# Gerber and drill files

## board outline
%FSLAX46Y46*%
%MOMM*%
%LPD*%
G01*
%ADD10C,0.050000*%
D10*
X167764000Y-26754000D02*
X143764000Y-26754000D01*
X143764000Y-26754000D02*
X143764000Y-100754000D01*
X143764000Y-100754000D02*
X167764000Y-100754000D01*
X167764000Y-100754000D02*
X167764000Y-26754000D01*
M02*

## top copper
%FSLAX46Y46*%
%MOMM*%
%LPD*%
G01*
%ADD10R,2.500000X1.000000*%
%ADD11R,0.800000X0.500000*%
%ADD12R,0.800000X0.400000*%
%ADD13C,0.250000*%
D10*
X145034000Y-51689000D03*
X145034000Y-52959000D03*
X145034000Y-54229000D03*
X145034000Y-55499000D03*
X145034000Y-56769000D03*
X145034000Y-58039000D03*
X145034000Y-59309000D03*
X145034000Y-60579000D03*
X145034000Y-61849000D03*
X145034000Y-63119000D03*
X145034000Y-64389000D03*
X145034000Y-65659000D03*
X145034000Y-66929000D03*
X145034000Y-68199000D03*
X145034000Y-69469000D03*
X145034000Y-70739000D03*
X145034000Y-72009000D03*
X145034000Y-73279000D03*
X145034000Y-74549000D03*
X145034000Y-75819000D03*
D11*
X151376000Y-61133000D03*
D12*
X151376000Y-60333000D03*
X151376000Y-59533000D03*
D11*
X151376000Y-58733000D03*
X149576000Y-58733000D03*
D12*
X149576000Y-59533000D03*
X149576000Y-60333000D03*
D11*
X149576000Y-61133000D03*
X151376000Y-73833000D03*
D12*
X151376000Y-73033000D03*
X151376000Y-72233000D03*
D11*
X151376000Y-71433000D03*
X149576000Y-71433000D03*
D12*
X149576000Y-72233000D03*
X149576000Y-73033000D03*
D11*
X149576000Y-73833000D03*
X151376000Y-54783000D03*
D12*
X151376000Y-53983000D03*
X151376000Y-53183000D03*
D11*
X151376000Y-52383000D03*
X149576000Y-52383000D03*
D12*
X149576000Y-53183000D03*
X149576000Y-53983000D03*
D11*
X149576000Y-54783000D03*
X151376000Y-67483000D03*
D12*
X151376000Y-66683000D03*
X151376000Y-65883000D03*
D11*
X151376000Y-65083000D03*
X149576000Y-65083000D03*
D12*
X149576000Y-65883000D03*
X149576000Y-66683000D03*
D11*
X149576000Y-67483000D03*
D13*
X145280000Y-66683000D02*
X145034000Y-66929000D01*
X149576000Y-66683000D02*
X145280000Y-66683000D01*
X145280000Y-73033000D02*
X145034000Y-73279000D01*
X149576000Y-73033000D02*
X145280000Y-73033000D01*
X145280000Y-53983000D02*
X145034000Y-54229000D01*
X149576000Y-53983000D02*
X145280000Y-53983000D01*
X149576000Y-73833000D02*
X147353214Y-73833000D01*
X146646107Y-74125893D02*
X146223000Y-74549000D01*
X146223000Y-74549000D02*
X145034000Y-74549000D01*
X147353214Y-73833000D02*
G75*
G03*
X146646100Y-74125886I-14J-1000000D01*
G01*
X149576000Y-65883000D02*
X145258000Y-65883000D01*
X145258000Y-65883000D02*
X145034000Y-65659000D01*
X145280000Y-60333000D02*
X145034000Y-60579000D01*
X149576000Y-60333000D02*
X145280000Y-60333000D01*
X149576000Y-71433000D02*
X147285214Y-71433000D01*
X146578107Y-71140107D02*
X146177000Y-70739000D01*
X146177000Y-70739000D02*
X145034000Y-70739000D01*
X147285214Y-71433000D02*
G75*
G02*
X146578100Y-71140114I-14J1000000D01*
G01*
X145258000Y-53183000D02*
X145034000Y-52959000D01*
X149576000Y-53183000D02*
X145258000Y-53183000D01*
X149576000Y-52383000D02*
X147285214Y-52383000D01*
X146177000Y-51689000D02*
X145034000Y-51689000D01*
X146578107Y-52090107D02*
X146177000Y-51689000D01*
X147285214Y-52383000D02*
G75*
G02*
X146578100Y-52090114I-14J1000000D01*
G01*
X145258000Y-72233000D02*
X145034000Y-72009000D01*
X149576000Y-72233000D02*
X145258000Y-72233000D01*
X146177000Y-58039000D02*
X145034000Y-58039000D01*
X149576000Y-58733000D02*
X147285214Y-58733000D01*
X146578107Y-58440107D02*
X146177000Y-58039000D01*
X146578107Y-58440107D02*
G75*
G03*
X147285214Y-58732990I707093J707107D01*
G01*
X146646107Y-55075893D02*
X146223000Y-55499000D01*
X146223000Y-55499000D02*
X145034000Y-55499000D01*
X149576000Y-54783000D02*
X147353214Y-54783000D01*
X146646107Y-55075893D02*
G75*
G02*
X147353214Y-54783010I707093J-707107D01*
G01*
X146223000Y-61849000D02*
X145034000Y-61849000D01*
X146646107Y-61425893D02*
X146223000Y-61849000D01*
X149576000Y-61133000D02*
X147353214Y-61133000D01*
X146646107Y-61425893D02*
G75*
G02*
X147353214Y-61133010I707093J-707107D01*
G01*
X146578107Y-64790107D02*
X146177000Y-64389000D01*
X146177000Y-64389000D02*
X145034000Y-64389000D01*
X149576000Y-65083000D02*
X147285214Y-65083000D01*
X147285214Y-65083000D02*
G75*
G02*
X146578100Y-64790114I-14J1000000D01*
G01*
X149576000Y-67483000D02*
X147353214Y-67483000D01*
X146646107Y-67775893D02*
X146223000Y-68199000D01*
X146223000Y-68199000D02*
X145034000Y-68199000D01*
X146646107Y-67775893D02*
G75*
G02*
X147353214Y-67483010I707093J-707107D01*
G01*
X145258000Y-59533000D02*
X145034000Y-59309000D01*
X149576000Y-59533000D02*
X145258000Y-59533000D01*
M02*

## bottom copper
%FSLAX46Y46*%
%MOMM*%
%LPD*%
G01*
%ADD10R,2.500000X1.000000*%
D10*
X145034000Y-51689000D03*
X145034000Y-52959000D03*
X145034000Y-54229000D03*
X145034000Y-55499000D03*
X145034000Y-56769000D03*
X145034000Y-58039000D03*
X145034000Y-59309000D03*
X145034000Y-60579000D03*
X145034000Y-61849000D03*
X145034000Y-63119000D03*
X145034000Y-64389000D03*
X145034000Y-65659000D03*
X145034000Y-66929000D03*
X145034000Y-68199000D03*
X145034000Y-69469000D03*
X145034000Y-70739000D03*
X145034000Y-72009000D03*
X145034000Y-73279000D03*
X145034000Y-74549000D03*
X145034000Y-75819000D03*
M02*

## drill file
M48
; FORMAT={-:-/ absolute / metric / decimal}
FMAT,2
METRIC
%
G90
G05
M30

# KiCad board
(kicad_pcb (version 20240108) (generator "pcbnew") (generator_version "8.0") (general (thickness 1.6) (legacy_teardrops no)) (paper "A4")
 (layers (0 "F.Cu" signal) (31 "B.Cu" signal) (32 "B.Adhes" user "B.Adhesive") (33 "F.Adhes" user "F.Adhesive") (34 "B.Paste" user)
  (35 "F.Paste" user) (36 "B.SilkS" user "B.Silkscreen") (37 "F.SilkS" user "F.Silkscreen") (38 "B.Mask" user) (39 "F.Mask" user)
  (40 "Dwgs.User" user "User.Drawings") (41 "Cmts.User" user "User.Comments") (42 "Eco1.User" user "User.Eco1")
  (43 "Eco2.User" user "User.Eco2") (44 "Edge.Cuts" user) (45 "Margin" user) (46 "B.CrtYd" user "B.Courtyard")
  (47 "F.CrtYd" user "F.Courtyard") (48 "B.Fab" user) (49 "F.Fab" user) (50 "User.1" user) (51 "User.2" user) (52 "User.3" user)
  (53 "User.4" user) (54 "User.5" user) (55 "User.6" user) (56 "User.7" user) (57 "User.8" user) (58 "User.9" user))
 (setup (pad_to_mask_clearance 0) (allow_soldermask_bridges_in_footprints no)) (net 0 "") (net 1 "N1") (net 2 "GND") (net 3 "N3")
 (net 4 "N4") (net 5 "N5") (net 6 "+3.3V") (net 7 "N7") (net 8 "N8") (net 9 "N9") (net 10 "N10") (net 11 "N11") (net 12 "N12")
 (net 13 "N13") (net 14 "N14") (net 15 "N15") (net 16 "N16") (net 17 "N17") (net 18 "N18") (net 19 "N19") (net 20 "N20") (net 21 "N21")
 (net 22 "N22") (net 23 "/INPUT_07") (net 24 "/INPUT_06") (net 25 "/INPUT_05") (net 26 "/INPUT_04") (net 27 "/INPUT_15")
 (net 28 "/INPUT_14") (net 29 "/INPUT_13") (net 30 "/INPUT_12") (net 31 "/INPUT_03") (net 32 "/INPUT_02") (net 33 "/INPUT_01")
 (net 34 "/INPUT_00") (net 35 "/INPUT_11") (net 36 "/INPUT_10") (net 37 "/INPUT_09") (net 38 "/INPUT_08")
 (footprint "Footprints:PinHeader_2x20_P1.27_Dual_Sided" (layer "F.Cu") (at 145.034 63.754)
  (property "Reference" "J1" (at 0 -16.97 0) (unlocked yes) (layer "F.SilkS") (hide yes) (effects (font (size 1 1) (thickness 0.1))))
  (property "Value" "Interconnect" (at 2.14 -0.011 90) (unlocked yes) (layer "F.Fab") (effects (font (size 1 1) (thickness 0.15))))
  (pad "1" smd rect (at 0 -12.065 180) (size 2.5 1) (layers "F.Cu" "F.Paste" "F.Mask") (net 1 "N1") (thermal_bridge_angle 45))
  (pad "2" smd rect (at 0 -12.065 180) (size 2.5 1) (layers "B.Cu" "B.Paste" "B.Mask") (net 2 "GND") (thermal_bridge_angle 45))
  (pad "3" smd rect (at 0 -10.795 180) (size 2.5 1) (layers "F.Cu" "F.Paste" "F.Mask") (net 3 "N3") (thermal_bridge_angle 45))
  (pad "4" smd rect (at 0 -10.795 180) (size 2.5 1) (layers "B.Cu" "B.Paste" "B.Mask") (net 2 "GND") (thermal_bridge_angle 45))
  (pad "5" smd rect (at 0 -9.525 180) (size 2.5 1) (layers "F.Cu" "F.Paste" "F.Mask") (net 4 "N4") (thermal_bridge_angle 45))
  (pad "6" smd rect (at 0 -9.525 180) (size 2.5 1) (layers "B.Cu" "B.Paste" "B.Mask") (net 2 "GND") (thermal_bridge_angle 45))
  (pad "7" smd rect (at 0 -8.255 180) (size 2.5 1) (layers "F.Cu" "F.Paste" "F.Mask") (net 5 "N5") (thermal_bridge_angle 45))
  (pad "8" smd rect (at 0 -8.255 180) (size 2.5 1) (layers "B.Cu" "B.Paste" "B.Mask") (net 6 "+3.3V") (thermal_bridge_angle 45))
  (pad "9" smd rect (at 0 -6.985 180) (size 2.5 1) (layers "F.Cu" "F.Paste" "F.Mask") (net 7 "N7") (thermal_bridge_angle 45))
  (pad "10" smd rect (at 0 -6.985 180) (size 2.5 1) (layers "B.Cu" "B.Paste" "B.Mask") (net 2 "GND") (thermal_bridge_angle 45))
  (pad "11" smd rect (at 0 -5.715 180) (size 2.5 1) (layers "F.Cu" "F.Paste" "F.Mask") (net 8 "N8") (thermal_bridge_angle 45))
  (pad "12" smd rect (at 0 -5.715 180) (size 2.5 1) (layers "B.Cu" "B.Paste" "B.Mask") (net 2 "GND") (thermal_bridge_angle 45))
  (pad "13" smd rect (at 0 -4.445 180) (size 2.5 1) (layers "F.Cu" "F.Paste" "F.Mask") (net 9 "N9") (thermal_bridge_angle 45))
  (pad "14" smd rect (at 0 -4.445 180) (size 2.5 1) (layers "B.Cu" "B.Paste" "B.Mask") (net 2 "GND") (thermal_bridge_angle 45))
  (pad "15" smd rect (at 0 -3.175 180) (size 2.5 1) (layers "F.Cu" "F.Paste" "F.Mask") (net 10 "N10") (thermal_bridge_angle 45))
  (pad "16" smd rect (at 0 -3.175 180) (size 2.5 1) (layers "B.Cu" "B.Paste" "B.Mask") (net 2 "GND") (thermal_bridge_angle 45))
  (pad "17" smd rect (at 0 -1.905 180) (size 2.5 1) (layers "F.Cu" "F.Paste" "F.Mask") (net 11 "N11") (thermal_bridge_angle 45))
  (pad "18" smd rect (at 0 -1.905 180) (size 2.5 1) (layers "B.Cu" "B.Paste" "B.Mask") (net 6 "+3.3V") (thermal_bridge_angle 45))
  (pad "19" smd rect (at 0 -0.635 180) (size 2.5 1) (layers "F.Cu" "F.Paste" "F.Mask") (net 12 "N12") (thermal_bridge_angle 45))
  (pad "20" smd rect (at 0 -0.635 180) (size 2.5 1) (layers "B.Cu" "B.Paste" "B.Mask") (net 2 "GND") (thermal_bridge_angle 45))
  (pad "21" smd rect (at 0 0.635 180) (size 2.5 1) (layers "F.Cu" "F.Paste" "F.Mask") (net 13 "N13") (thermal_bridge_angle 45))
  (pad "22" smd rect (at 0 0.635 180) (size 2.5 1) (layers "B.Cu" "B.Paste" "B.Mask") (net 2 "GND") (thermal_bridge_angle 45))
  (pad "23" smd rect (at 0 1.905 180) (size 2.5 1) (layers "F.Cu" "F.Paste" "F.Mask") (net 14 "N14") (thermal_bridge_angle 45))
  (pad "24" smd rect (at 0 1.905 180) (size 2.5 1) (layers "B.Cu" "B.Paste" "B.Mask") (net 2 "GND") (thermal_bridge_angle 45))
  (pad "25" smd rect (at 0 3.175 180) (size 2.5 1) (layers "F.Cu" "F.Paste" "F.Mask") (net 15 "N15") (thermal_bridge_angle 45))
  (pad "26" smd rect (at 0 3.175 180) (size 2.5 1) (layers "B.Cu" "B.Paste" "B.Mask") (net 2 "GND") (thermal_bridge_angle 45))
  (pad "27" smd rect (at 0 4.445 180) (size 2.5 1) (layers "F.Cu" "F.Paste" "F.Mask") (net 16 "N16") (thermal_bridge_angle 45))
  (pad "28" smd rect (at 0 4.445 180) (size 2.5 1) (layers "B.Cu" "B.Paste" "B.Mask") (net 6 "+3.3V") (thermal_bridge_angle 45))
  (pad "29" smd rect (at 0 5.715 180) (size 2.5 1) (layers "F.Cu" "F.Paste" "F.Mask") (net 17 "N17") (thermal_bridge_angle 45))
  (pad "30" smd rect (at 0 5.715 180) (size 2.5 1) (layers "B.Cu" "B.Paste" "B.Mask") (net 2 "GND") (thermal_bridge_angle 45))
  (pad "31" smd rect (at 0 6.985 180) (size 2.5 1) (layers "F.Cu" "F.Paste" "F.Mask") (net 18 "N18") (thermal_bridge_angle 45))
  (pad "32" smd rect (at 0 6.985 180) (size 2.5 1) (layers "B.Cu" "B.Paste" "B.Mask") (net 2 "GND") (thermal_bridge_angle 45))
  (pad "33" smd rect (at 0 8.255 180) (size 2.5 1) (layers "F.Cu" "F.Paste" "F.Mask") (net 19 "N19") (thermal_bridge_angle 45))
  (pad "34" smd rect (at 0 8.255 180) (size 2.5 1) (layers "B.Cu" "B.Paste" "B.Mask") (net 2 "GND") (thermal_bridge_angle 45))
  (pad "35" smd rect (at 0 9.525 180) (size 2.5 1) (layers "F.Cu" "F.Paste" "F.Mask") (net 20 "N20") (thermal_bridge_angle 45))
  (pad "36" smd rect (at 0 9.525 180) (size 2.5 1) (layers "B.Cu" "B.Paste" "B.Mask") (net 2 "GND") (thermal_bridge_angle 45))
  (pad "37" smd rect (at 0 10.795 180) (size 2.5 1) (layers "F.Cu" "F.Paste" "F.Mask") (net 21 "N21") (thermal_bridge_angle 45))
  (pad "38" smd rect (at 0 10.795 180) (size 2.5 1) (layers "B.Cu" "B.Paste" "B.Mask") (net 6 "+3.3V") (thermal_bridge_angle 45))
  (pad "39" smd rect (at 0 12.065 180) (size 2.5 1) (layers "F.Cu" "F.Paste" "F.Mask") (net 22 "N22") (thermal_bridge_angle 45))
  (pad "40" smd rect (at 0 12.065 180) (size 2.5 1) (layers "B.Cu" "B.Paste" "B.Mask") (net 2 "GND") (thermal_bridge_angle 45)))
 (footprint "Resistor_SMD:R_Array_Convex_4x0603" (layer "F.Cu") (at 150.476 59.933 180)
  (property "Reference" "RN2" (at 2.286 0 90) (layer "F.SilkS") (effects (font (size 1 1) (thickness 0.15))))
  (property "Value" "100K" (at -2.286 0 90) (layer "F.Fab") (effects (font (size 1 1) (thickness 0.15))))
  (pad "1" smd rect (at -0.9 -1.2 180) (size 0.8 0.5) (layers "F.Cu" "F.Paste" "F.Mask") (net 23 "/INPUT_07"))
  (pad "2" smd rect (at -0.9 -0.4 180) (size 0.8 0.4) (layers "F.Cu" "F.Paste" "F.Mask") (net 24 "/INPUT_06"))
  (pad "3" smd rect (at -0.9 0.4 180) (size 0.8 0.4) (layers "F.Cu" "F.Paste" "F.Mask") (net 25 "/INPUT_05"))
  (pad "4" smd rect (at -0.9 1.2 180) (size 0.8 0.5) (layers "F.Cu" "F.Paste" "F.Mask") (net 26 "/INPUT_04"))
  (pad "5" smd rect (at 0.9 1.2 180) (size 0.8 0.5) (layers "F.Cu" "F.Paste" "F.Mask") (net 8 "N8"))
  (pad "6" smd rect (at 0.9 0.4 180) (size 0.8 0.4) (layers "F.Cu" "F.Paste" "F.Mask") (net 9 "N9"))
  (pad "7" smd rect (at 0.9 -0.4 180) (size 0.8 0.4) (layers "F.Cu" "F.Paste" "F.Mask") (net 10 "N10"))
  (pad "8" smd rect (at 0.9 -1.2 180) (size 0.8 0.5) (layers "F.Cu" "F.Paste" "F.Mask") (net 11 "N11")))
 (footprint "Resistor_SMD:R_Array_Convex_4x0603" (layer "F.Cu") (at 150.476 72.633 180)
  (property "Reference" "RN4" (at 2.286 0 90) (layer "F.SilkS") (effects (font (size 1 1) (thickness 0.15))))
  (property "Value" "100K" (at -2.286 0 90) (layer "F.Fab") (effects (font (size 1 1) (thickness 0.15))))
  (pad "1" smd rect (at -0.9 -1.2 180) (size 0.8 0.5) (layers "F.Cu" "F.Paste" "F.Mask") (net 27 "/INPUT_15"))
  (pad "2" smd rect (at -0.9 -0.4 180) (size 0.8 0.4) (layers "F.Cu" "F.Paste" "F.Mask") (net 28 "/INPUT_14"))
  (pad "3" smd rect (at -0.9 0.4 180) (size 0.8 0.4) (layers "F.Cu" "F.Paste" "F.Mask") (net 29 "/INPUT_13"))
  (pad "4" smd rect (at -0.9 1.2 180) (size 0.8 0.5) (layers "F.Cu" "F.Paste" "F.Mask") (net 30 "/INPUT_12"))
  (pad "5" smd rect (at 0.9 1.2 180) (size 0.8 0.5) (layers "F.Cu" "F.Paste" "F.Mask") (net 18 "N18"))
  (pad "6" smd rect (at 0.9 0.4 180) (size 0.8 0.4) (layers "F.Cu" "F.Paste" "F.Mask") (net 19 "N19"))
  (pad "7" smd rect (at 0.9 -0.4 180) (size 0.8 0.4) (layers "F.Cu" "F.Paste" "F.Mask") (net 20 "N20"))
  (pad "8" smd rect (at 0.9 -1.2 180) (size 0.8 0.5) (layers "F.Cu" "F.Paste" "F.Mask") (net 21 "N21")))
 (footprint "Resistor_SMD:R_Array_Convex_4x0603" (layer "F.Cu") (at 150.476 53.583 180)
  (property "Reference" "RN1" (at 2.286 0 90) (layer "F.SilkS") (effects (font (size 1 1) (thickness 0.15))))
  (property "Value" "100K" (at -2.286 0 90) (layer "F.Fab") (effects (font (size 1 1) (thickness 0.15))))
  (pad "1" smd rect (at -0.9 -1.2 180) (size 0.8 0.5) (layers "F.Cu" "F.Paste" "F.Mask") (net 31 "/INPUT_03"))
  (pad "2" smd rect (at -0.9 -0.4 180) (size 0.8 0.4) (layers "F.Cu" "F.Paste" "F.Mask") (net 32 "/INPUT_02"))
  (pad "3" smd rect (at -0.9 0.4 180) (size 0.8 0.4) (layers "F.Cu" "F.Paste" "F.Mask") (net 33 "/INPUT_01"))
  (pad "4" smd rect (at -0.9 1.2 180) (size 0.8 0.5) (layers "F.Cu" "F.Paste" "F.Mask") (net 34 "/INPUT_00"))
  (pad "5" smd rect (at 0.9 1.2 180) (size 0.8 0.5) (layers "F.Cu" "F.Paste" "F.Mask") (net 1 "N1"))
  (pad "6" smd rect (at 0.9 0.4 180) (size 0.8 0.4) (layers "F.Cu" "F.Paste" "F.Mask") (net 3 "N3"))
  (pad "7" smd rect (at 0.9 -0.4 180) (size 0.8 0.4) (layers "F.Cu" "F.Paste" "F.Mask") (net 4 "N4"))
  (pad "8" smd rect (at 0.9 -1.2 180) (size 0.8 0.5) (layers "F.Cu" "F.Paste" "F.Mask") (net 5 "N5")))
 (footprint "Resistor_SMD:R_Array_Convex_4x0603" (layer "F.Cu") (at 150.476 66.283 180)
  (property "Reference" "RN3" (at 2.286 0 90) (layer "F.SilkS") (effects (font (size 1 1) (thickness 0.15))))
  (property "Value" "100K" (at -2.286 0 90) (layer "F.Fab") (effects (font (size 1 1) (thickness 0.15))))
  (pad "1" smd rect (at -0.9 -1.2 180) (size 0.8 0.5) (layers "F.Cu" "F.Paste" "F.Mask") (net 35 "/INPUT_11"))
  (pad "2" smd rect (at -0.9 -0.4 180) (size 0.8 0.4) (layers "F.Cu" "F.Paste" "F.Mask") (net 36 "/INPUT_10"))
  (pad "3" smd rect (at -0.9 0.4 180) (size 0.8 0.4) (layers "F.Cu" "F.Paste" "F.Mask") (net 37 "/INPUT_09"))
  (pad "4" smd rect (at -0.9 1.2 180) (size 0.8 0.5) (layers "F.Cu" "F.Paste" "F.Mask") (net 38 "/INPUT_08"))
  (pad "5" smd rect (at 0.9 1.2 180) (size 0.8 0.5) (layers "F.Cu" "F.Paste" "F.Mask") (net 13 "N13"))
  (pad "6" smd rect (at 0.9 0.4 180) (size 0.8 0.4) (layers "F.Cu" "F.Paste" "F.Mask") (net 14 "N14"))
  (pad "7" smd rect (at 0.9 -0.4 180) (size 0.8 0.4) (layers "F.Cu" "F.Paste" "F.Mask") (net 15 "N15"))
  (pad "8" smd rect (at 0.9 -1.2 180) (size 0.8 0.5) (layers "F.Cu" "F.Paste" "F.Mask") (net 16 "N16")))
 (gr_line (start 167.764 26.754) (end 143.764 26.754) (stroke (width 0.05) (type default)) (layer "Edge.Cuts"))
 (gr_line (start 143.764 26.754) (end 143.764 100.754) (stroke (width 0.05) (type default)) (layer "Edge.Cuts"))
 (gr_line (start 143.764 100.754) (end 167.764 100.754) (stroke (width 0.05) (type default)) (layer "Edge.Cuts"))
 (gr_line (start 167.764 100.754) (end 167.764 26.754) (stroke (width 0.05) (type default)) (layer "Edge.Cuts"))
 (segment (start 145.28 66.683) (end 145.034 66.929) (width 0.25) (layer "F.Cu") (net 15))
 (segment (start 149.576 66.683) (end 145.28 66.683) (width 0.25) (layer "F.Cu") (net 15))
 (segment (start 145.28 73.033) (end 145.034 73.279) (width 0.25) (layer "F.Cu") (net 20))
 (segment (start 149.576 73.033) (end 145.28 73.033) (width 0.25) (layer "F.Cu") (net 20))
 (segment (start 145.28 53.983) (end 145.034 54.229) (width 0.25) (layer "F.Cu") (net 4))
 (segment (start 149.576 53.983) (end 145.28 53.983) (width 0.25) (layer "F.Cu") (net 4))
 (segment (start 149.576 73.833) (end 147.353214 73.833) (width 0.25) (layer "F.Cu") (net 21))
 (segment (start 146.646107 74.125893) (end 146.223 74.549) (width 0.25) (layer "F.Cu") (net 21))
 (segment (start 146.223 74.549) (end 145.034 74.549) (width 0.25) (layer "F.Cu") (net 21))
 (arc (start 147.353214 73.833) (mid 146.970531 73.90912) (end 146.646107 74.125893) (width 0.25) (layer "F.Cu") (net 21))
 (segment (start 149.576 65.883) (end 145.258 65.883) (width 0.25) (layer "F.Cu") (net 14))
 (segment (start 145.258 65.883) (end 145.034 65.659) (width 0.25) (layer "F.Cu") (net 14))
 (segment (start 145.28 60.333) (end 145.034 60.579) (width 0.25) (layer "F.Cu") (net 10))
 (segment (start 149.576 60.333) (end 145.28 60.333) (width 0.25) (layer "F.Cu") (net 10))
 (segment (start 149.576 71.433) (end 147.285214 71.433) (width 0.25) (layer "F.Cu") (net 18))
 (segment (start 146.578107 71.140107) (end 146.177 70.739) (width 0.25) (layer "F.Cu") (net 18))
 (segment (start 146.177 70.739) (end 145.034 70.739) (width 0.25) (layer "F.Cu") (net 18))
 (arc (start 147.285214 71.433) (mid 146.902531 71.35688) (end 146.578107 71.140107) (width 0.25) (layer "F.Cu") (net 18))
 (segment (start 145.258 53.183) (end 145.034 52.959) (width 0.25) (layer "F.Cu") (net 3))
 (segment (start 149.576 53.183) (end 145.258 53.183) (width 0.25) (layer "F.Cu") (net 3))
 (segment (start 149.576 52.383) (end 147.285214 52.383) (width 0.25) (layer "F.Cu") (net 1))
 (segment (start 146.177 51.689) (end 145.034 51.689) (width 0.25) (layer "F.Cu") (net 1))
 (segment (start 146.578107 52.090107) (end 146.177 51.689) (width 0.25) (layer "F.Cu") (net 1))
 (arc (start 147.285214 52.383) (mid 146.902531 52.30688) (end 146.578107 52.090107) (width 0.25) (layer "F.Cu") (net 1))
 (segment (start 145.258 72.233) (end 145.034 72.009) (width 0.25) (layer "F.Cu") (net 19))
 (segment (start 149.576 72.233) (end 145.258 72.233) (width 0.25) (layer "F.Cu") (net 19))
 (segment (start 146.177 58.039) (end 145.034 58.039) (width 0.25) (layer "F.Cu") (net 8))
 (segment (start 149.576 58.733) (end 147.285214 58.733) (width 0.25) (layer "F.Cu") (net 8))
 (segment (start 146.578107 58.440107) (end 146.177 58.039) (width 0.25) (layer "F.Cu") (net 8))
 (arc (start 146.578107 58.440107) (mid 146.90253 58.65688) (end 147.285214 58.733) (width 0.25) (layer "F.Cu") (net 8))
 (segment (start 146.646107 55.075893) (end 146.223 55.499) (width 0.25) (layer "F.Cu") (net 5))
 (segment (start 146.223 55.499) (end 145.034 55.499) (width 0.25) (layer "F.Cu") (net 5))
 (segment (start 149.576 54.783) (end 147.353214 54.783) (width 0.25) (layer "F.Cu") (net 5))
 (arc (start 146.646107 55.075893) (mid 146.97053 54.85912) (end 147.353214 54.783) (width 0.25) (layer "F.Cu") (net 5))
 (segment (start 146.223 61.849) (end 145.034 61.849) (width 0.25) (layer "F.Cu") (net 11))
 (segment (start 146.646107 61.425893) (end 146.223 61.849) (width 0.25) (layer "F.Cu") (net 11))
 (segment (start 149.576 61.133) (end 147.353214 61.133) (width 0.25) (layer "F.Cu") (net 11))
 (arc (start 146.646107 61.425893) (mid 146.97053 61.20912) (end 147.353214 61.133) (width 0.25) (layer "F.Cu") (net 11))
 (segment (start 146.578107 64.790107) (end 146.177 64.389) (width 0.25) (layer "F.Cu") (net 13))
 (segment (start 146.177 64.389) (end 145.034 64.389) (width 0.25) (layer "F.Cu") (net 13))
 (segment (start 149.576 65.083) (end 147.285214 65.083) (width 0.25) (layer "F.Cu") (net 13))
 (arc (start 147.285214 65.083) (mid 146.902531 65.00688) (end 146.578107 64.790107) (width 0.25) (layer "F.Cu") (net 13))
 (segment (start 149.576 67.483) (end 147.353214 67.483) (width 0.25) (layer "F.Cu") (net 16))
 (segment (start 146.646107 67.775893) (end 146.223 68.199) (width 0.25) (layer "F.Cu") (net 16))
 (segment (start 146.223 68.199) (end 145.034 68.199) (width 0.25) (layer "F.Cu") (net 16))
 (arc (start 146.646107 67.775893) (mid 146.97053 67.55912) (end 147.353214 67.483) (width 0.25) (layer "F.Cu") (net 16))
 (segment (start 145.258 59.533) (end 145.034 59.309) (width 0.25) (layer "F.Cu") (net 9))
 (segment (start 149.576 59.533) (end 145.258 59.533) (width 0.25) (layer "F.Cu") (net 9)))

